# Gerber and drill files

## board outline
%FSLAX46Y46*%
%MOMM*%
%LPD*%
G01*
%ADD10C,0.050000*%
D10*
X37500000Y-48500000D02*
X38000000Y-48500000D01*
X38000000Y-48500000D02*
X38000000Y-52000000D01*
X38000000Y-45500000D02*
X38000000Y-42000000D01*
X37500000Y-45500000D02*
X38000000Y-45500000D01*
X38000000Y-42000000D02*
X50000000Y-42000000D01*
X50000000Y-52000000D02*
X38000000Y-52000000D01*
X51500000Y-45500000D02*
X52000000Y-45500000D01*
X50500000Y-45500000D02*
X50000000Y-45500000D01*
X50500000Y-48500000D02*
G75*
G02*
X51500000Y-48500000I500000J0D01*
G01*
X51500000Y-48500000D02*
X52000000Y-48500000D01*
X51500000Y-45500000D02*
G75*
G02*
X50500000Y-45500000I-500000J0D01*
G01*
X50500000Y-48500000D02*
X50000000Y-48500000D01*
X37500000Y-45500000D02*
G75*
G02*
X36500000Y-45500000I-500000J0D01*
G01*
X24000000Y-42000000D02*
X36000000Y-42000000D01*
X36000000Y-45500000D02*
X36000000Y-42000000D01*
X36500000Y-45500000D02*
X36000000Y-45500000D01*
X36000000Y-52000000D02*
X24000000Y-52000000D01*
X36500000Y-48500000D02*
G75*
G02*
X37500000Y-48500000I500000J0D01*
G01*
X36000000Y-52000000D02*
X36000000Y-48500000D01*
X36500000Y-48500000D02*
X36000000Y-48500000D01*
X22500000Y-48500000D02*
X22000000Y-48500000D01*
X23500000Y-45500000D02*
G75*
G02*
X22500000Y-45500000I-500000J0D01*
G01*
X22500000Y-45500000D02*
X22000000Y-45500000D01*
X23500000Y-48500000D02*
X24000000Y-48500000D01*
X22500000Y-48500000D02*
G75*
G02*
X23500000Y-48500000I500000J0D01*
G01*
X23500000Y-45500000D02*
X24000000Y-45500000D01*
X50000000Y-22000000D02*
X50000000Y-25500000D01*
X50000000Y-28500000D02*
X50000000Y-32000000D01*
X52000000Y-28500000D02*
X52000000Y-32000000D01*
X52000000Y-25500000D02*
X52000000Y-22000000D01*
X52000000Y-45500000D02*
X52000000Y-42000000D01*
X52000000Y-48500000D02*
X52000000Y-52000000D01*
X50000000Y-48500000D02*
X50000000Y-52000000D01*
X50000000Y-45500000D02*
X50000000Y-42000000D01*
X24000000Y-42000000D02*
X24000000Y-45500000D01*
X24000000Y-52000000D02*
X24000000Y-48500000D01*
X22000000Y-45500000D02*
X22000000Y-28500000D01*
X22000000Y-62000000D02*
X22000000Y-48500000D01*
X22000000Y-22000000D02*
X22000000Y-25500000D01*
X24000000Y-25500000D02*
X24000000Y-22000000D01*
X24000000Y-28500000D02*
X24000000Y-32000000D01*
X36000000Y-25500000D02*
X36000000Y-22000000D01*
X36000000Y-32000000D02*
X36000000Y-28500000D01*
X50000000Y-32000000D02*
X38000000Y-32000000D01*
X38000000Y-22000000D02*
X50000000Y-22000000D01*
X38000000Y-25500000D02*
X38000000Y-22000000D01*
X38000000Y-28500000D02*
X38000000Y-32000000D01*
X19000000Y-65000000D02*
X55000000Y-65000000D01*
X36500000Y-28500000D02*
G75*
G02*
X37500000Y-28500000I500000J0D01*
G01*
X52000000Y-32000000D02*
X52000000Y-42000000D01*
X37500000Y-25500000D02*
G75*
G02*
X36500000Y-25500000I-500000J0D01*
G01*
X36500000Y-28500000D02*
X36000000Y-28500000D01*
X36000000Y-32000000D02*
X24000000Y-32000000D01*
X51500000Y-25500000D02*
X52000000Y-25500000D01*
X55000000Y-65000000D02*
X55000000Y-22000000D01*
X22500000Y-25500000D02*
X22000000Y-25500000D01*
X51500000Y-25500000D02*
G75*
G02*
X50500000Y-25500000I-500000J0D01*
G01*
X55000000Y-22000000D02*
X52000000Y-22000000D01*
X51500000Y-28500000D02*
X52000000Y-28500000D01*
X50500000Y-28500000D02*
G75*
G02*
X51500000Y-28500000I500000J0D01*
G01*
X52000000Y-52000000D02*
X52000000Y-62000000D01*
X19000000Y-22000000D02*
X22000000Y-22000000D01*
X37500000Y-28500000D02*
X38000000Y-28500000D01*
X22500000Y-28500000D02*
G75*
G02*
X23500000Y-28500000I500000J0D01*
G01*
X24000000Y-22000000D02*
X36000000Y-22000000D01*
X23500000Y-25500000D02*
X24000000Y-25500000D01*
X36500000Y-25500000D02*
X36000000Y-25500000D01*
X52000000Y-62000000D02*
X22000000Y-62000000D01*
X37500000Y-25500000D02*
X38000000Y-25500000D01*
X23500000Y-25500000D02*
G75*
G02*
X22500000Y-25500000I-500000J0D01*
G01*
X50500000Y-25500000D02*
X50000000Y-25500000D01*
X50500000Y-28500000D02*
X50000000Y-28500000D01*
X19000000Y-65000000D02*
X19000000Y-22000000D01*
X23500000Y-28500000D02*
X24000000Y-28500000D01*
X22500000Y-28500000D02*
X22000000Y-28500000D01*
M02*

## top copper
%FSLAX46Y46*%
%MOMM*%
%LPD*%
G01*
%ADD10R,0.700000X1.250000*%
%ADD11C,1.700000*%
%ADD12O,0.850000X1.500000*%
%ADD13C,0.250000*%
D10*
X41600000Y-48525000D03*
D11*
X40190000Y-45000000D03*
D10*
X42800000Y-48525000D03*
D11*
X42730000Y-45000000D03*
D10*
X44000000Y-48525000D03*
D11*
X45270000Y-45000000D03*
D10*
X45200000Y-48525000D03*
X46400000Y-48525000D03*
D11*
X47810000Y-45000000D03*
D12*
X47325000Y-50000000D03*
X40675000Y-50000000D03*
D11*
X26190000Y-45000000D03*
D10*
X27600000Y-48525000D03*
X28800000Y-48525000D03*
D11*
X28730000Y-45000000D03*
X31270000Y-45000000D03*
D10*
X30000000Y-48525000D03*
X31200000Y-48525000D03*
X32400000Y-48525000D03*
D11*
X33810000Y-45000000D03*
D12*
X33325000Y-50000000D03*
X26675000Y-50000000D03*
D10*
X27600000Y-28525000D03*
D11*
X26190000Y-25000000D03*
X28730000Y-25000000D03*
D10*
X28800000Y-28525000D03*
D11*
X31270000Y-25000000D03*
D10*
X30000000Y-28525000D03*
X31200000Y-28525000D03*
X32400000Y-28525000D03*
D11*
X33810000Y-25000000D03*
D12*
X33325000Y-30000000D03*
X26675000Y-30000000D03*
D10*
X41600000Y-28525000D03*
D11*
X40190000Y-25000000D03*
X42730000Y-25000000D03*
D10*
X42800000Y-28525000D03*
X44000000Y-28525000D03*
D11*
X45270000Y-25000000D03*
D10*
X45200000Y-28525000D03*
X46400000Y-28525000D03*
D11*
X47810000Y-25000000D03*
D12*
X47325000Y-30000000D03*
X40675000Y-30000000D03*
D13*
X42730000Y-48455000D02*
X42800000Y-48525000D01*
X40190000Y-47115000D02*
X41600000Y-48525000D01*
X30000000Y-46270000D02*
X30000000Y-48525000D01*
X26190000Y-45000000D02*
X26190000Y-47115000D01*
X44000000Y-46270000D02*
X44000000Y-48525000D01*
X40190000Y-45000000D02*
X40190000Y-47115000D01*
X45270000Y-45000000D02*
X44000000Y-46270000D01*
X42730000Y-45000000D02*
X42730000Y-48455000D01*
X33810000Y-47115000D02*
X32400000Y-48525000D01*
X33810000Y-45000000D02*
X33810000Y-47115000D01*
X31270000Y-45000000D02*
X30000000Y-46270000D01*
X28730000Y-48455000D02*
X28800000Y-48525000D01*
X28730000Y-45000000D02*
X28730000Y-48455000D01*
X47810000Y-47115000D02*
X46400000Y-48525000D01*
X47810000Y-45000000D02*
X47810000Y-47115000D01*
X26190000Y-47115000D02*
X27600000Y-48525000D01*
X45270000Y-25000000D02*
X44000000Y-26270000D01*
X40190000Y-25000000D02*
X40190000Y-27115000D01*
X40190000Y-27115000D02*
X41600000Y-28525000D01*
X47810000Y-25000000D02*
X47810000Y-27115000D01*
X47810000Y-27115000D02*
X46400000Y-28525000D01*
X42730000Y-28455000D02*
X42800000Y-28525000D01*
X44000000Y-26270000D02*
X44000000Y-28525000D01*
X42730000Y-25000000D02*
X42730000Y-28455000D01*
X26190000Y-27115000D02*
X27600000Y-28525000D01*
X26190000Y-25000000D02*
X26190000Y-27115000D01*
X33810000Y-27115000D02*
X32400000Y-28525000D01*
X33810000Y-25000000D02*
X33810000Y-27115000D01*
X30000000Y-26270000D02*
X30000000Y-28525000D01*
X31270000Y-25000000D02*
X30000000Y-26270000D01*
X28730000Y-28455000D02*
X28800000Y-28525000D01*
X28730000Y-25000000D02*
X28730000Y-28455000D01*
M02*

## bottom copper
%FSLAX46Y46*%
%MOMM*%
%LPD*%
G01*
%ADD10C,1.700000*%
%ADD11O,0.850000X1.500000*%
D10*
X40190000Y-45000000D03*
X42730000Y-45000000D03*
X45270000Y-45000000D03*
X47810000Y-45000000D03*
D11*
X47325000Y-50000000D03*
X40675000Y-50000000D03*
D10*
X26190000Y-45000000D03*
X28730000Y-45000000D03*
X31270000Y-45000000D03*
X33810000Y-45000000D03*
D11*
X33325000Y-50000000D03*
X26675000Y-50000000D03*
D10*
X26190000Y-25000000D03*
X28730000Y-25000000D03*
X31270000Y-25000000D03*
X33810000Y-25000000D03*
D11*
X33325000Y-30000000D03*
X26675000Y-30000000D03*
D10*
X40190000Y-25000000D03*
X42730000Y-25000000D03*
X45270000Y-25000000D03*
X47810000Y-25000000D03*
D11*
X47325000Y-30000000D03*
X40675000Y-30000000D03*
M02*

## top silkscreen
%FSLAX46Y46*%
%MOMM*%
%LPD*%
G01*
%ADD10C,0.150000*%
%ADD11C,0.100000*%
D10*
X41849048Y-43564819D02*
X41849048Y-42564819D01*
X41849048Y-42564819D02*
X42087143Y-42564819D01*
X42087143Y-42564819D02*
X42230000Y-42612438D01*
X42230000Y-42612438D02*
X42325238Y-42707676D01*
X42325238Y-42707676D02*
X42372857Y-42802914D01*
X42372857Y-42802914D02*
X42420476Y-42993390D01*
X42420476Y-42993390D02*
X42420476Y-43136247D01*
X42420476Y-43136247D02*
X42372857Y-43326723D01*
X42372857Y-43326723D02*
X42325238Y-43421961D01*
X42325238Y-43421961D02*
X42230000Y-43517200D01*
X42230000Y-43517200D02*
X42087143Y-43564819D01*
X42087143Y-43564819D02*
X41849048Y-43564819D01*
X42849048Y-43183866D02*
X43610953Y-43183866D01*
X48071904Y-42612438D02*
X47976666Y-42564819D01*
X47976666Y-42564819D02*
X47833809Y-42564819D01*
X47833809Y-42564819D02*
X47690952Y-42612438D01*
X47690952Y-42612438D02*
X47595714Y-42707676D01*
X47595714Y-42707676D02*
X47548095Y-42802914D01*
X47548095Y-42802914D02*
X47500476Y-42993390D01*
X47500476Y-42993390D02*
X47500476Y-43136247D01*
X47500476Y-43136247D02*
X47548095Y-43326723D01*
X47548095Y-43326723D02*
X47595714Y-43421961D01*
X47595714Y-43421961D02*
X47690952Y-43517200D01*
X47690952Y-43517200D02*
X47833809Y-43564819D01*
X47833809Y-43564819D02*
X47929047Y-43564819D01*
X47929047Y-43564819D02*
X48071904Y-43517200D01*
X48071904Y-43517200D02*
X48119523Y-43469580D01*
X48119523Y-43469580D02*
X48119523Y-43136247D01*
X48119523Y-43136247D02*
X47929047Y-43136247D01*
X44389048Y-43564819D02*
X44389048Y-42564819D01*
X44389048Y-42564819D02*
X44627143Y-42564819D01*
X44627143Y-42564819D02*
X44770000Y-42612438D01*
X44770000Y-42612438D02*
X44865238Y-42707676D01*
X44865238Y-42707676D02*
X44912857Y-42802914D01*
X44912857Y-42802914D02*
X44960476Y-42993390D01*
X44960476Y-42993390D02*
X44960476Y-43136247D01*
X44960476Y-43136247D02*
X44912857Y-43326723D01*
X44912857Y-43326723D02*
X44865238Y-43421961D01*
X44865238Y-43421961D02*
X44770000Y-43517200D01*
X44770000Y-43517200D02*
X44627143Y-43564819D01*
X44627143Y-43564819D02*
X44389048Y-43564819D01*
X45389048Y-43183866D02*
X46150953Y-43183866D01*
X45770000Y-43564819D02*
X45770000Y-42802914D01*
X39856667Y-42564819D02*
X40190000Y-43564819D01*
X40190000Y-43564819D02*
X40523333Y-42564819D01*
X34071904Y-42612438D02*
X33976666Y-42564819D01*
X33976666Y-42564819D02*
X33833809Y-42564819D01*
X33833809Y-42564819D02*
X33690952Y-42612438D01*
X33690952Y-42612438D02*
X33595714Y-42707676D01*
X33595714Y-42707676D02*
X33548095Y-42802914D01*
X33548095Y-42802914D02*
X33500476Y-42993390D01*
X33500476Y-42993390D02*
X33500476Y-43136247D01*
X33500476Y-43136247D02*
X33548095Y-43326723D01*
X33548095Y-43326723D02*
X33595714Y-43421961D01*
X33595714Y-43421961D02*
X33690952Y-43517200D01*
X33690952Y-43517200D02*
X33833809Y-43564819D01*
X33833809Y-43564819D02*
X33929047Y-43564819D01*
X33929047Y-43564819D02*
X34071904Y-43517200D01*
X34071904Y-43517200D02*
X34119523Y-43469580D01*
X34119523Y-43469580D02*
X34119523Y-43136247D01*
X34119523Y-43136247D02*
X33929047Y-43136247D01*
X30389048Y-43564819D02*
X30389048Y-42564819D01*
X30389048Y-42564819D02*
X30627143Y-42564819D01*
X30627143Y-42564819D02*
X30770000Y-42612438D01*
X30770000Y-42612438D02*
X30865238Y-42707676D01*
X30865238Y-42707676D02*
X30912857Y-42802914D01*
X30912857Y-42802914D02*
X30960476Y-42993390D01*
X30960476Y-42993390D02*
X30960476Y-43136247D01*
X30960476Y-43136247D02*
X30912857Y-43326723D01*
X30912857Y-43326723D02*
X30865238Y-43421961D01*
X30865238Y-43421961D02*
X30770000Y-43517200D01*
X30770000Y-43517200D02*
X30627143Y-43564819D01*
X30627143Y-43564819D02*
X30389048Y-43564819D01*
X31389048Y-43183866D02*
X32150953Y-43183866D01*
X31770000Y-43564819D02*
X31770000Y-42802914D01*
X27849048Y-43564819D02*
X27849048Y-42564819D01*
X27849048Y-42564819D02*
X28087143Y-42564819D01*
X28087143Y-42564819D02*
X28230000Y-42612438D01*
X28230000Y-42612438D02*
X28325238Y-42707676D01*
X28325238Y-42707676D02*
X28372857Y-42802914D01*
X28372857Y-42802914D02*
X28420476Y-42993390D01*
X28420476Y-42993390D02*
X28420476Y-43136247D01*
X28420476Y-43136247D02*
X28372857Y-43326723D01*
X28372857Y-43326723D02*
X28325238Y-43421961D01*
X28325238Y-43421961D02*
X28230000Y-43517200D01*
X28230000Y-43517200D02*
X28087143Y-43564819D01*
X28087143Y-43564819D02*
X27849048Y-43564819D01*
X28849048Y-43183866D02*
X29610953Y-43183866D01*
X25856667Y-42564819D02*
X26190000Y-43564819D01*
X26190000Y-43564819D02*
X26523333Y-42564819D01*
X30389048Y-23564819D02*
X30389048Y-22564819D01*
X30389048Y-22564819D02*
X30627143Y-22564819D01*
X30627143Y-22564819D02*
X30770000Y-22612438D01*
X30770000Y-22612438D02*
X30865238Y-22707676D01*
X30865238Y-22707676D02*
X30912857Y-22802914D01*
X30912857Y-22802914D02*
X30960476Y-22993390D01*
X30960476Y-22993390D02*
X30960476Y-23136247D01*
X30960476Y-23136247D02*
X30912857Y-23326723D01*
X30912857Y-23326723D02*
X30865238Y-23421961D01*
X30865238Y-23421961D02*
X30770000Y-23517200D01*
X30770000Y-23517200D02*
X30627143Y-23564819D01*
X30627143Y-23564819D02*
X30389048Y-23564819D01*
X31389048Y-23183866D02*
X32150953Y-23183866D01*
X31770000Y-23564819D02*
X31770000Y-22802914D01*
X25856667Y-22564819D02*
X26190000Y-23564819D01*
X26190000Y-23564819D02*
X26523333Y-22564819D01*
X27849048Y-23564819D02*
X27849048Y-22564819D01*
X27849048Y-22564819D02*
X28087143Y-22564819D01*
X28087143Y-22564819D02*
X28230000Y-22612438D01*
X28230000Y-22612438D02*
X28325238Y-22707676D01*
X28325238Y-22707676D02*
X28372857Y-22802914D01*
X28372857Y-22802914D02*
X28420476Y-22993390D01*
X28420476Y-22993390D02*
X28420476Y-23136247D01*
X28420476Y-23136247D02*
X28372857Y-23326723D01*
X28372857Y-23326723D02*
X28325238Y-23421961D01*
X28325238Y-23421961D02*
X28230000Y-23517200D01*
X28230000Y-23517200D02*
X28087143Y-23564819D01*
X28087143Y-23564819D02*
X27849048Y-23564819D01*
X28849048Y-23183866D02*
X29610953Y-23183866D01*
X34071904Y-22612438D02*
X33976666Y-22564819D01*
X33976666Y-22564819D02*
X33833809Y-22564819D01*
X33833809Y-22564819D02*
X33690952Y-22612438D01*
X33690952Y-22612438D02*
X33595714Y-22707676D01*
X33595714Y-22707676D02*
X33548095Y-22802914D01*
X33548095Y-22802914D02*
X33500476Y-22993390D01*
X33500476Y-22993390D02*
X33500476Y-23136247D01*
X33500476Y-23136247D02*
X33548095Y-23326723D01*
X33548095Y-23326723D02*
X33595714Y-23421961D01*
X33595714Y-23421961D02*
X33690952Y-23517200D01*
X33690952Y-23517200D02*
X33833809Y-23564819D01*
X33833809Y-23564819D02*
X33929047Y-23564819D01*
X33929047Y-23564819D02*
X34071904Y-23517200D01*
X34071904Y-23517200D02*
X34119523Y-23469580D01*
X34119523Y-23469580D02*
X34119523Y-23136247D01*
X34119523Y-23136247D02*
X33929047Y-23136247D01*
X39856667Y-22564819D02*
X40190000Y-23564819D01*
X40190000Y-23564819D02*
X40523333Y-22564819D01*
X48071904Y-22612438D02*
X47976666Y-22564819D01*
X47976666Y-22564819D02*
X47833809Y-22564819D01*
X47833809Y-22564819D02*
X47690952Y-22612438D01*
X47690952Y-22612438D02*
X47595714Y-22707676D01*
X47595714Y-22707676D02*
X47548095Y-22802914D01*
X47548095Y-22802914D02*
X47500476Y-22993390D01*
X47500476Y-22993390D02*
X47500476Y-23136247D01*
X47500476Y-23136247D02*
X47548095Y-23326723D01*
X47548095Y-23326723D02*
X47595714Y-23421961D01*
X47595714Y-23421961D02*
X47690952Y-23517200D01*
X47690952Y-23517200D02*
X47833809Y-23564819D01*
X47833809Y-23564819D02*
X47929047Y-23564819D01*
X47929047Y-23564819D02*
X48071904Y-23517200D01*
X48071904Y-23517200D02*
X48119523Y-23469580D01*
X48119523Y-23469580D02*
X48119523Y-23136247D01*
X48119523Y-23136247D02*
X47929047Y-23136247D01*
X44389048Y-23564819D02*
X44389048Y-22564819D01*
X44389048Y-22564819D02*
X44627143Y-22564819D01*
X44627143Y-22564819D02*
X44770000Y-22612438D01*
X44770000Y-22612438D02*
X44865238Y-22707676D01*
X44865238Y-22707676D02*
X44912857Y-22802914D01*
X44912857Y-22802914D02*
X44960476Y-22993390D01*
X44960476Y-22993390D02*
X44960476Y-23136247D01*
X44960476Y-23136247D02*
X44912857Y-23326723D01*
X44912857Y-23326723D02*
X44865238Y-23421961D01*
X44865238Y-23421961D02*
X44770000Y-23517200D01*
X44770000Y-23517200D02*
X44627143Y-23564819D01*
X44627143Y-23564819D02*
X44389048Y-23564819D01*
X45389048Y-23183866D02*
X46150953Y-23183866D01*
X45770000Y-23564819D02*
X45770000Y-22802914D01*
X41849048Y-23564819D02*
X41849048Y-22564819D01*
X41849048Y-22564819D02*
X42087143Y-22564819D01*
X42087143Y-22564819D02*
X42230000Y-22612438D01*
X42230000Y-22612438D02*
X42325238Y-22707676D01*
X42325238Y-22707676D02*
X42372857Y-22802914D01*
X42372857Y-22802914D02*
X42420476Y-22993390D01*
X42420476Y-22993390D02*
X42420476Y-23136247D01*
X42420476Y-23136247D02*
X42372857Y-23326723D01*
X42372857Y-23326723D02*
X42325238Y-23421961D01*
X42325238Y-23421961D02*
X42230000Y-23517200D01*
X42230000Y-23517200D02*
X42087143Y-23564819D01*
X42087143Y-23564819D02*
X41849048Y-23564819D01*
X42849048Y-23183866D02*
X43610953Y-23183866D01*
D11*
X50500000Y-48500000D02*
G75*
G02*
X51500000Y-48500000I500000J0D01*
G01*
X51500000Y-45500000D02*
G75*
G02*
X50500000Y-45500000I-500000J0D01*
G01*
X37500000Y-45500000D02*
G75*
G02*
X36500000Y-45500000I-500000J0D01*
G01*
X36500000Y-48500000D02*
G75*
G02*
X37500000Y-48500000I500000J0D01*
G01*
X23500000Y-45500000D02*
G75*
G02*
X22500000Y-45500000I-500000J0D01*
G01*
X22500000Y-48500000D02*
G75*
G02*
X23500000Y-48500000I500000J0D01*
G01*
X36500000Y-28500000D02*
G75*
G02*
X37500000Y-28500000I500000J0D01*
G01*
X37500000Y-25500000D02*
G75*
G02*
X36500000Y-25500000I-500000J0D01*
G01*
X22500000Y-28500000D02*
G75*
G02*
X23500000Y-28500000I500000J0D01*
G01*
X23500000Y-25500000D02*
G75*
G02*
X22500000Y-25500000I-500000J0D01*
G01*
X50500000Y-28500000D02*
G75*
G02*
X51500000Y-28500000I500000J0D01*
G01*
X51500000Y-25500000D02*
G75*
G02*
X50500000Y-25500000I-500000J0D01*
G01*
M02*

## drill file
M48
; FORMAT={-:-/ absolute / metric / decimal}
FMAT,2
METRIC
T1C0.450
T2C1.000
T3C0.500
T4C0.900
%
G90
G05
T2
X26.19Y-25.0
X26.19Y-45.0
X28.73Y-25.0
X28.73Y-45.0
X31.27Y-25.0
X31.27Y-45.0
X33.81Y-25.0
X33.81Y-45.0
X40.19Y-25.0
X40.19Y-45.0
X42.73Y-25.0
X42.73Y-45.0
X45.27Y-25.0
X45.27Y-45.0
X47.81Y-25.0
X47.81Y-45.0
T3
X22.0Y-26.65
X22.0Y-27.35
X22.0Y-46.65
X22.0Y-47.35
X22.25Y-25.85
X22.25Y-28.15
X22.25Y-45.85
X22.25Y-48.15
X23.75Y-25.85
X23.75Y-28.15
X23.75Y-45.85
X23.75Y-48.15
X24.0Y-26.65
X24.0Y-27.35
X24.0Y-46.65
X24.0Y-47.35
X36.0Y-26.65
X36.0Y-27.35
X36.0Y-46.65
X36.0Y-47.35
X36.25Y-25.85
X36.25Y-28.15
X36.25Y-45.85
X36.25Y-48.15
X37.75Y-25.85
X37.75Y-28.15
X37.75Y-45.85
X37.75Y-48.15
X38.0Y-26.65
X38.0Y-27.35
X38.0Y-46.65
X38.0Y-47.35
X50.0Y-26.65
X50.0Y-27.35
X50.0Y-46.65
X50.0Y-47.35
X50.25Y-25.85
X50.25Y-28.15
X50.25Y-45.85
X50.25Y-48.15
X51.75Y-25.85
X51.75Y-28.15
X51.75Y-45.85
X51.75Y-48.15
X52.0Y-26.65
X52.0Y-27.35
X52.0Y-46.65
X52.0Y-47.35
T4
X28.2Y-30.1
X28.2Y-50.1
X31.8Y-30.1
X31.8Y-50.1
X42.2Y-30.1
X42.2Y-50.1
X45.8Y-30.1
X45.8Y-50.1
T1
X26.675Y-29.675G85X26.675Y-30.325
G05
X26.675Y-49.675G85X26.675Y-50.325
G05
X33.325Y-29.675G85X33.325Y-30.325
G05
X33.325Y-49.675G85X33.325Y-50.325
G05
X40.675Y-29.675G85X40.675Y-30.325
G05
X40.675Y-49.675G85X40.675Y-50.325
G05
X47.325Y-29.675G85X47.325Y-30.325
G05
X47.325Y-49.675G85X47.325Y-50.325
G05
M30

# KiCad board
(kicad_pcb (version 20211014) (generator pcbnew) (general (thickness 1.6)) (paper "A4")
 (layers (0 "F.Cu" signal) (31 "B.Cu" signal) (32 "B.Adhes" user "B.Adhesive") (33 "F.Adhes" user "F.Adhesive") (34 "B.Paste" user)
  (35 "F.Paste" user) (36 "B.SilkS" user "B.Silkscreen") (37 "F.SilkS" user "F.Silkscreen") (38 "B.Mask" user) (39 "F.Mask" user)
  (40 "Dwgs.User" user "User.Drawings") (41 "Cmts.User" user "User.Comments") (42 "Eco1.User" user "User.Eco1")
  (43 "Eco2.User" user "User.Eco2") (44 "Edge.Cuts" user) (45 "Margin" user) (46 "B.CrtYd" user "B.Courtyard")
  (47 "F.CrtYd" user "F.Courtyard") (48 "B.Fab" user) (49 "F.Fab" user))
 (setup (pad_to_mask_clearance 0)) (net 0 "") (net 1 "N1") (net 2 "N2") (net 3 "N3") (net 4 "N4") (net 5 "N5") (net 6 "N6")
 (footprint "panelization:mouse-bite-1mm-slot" (layer "F.Cu") (at 51 47 90)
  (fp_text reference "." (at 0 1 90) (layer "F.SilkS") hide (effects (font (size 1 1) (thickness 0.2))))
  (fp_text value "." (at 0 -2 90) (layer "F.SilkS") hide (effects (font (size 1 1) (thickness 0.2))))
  (fp_arc (start -1.5 -0.5) (mid -1 0) (end -1.5 0.5) (layer "F.SilkS") (width 0.1))
  (fp_arc (start 1.5 0.5) (mid 1 0) (end 1.5 -0.5) (layer "F.SilkS") (width 0.1))
  (pad "" np_thru_hole circle locked (at -1.15 -0.75 90) (size 0.5 0.5) (drill 0.5) (layers *.Cu *.Mask))
  (pad "" np_thru_hole circle locked (at -0.35 1 90) (size 0.5 0.5) (drill 0.5) (layers *.Cu *.Mask))
  (pad "" np_thru_hole circle locked (at -0.35 -1 90) (size 0.5 0.5) (drill 0.5) (layers *.Cu *.Mask))
  (pad "" np_thru_hole circle locked (at 0.35 -1 90) (size 0.5 0.5) (drill 0.5) (layers *.Cu *.Mask))
  (pad "" np_thru_hole circle locked (at 1.15 -0.75 90) (size 0.5 0.5) (drill 0.5) (layers *.Cu *.Mask))
  (pad "" np_thru_hole circle locked (at 1.15 0.75 90) (size 0.5 0.5) (drill 0.5) (layers *.Cu *.Mask))
  (pad "" np_thru_hole circle locked (at -1.15 0.75 90) (size 0.5 0.5) (drill 0.5) (layers *.Cu *.Mask))
  (pad "" np_thru_hole circle locked (at 0.35 1 90) (size 0.5 0.5) (drill 0.5) (layers *.Cu *.Mask)))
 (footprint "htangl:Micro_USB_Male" (layer "F.Cu") (at 44 50)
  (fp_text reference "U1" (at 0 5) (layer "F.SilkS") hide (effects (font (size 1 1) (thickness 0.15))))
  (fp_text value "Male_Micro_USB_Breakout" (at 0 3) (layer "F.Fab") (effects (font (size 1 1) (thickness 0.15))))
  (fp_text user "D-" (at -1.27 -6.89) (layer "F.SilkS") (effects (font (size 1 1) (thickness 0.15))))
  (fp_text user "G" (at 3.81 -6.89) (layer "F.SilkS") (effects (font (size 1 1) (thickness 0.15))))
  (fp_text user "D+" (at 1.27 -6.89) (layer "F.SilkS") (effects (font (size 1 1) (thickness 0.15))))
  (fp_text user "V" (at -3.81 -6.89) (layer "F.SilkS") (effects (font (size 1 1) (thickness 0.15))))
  (pad "" np_thru_hole circle (at -1.8 0.1) (size 0.9 0.9) (drill 0.9) (layers *.Cu *.Mask))
  (pad "" np_thru_hole circle (at 1.8 0.1) (size 0.9 0.9) (drill 0.9) (layers *.Cu *.Mask))
  (pad "1" smd rect (at -2.4 -1.475) (size 0.7 1.25) (layers "F.Cu" "F.Paste" "F.Mask"))
  (pad "1" thru_hole circle (at -3.81 -5) (size 1.7 1.7) (drill 1) (layers *.Cu *.Mask))
  (pad "2" smd rect (at -1.2 -1.475) (size 0.7 1.25) (layers "F.Cu" "F.Paste" "F.Mask"))
  (pad "2" thru_hole circle (at -1.27 -5) (size 1.7 1.7) (drill 1) (layers *.Cu *.Mask))
  (pad "3" smd rect (at 0 -1.475) (size 0.7 1.25) (layers "F.Cu" "F.Paste" "F.Mask"))
  (pad "3" thru_hole circle (at 1.27 -5) (size 1.7 1.7) (drill 1) (layers *.Cu *.Mask))
  (pad "4" smd rect (at 1.2 -1.475) (size 0.7 1.25) (layers "F.Cu" "F.Paste" "F.Mask"))
  (pad "5" smd rect (at 2.4 -1.475) (size 0.7 1.25) (layers "F.Cu" "F.Paste" "F.Mask"))
  (pad "5" thru_hole circle (at 3.81 -5) (size 1.7 1.7) (drill 1) (layers *.Cu *.Mask))
  (pad "6" thru_hole oval (at 3.325 0) (size 0.85 1.5) (drill oval 0.45 1.1) (layers *.Cu *.Mask))
  (pad "6" thru_hole oval (at -3.325 0) (size 0.85 1.5) (drill oval 0.45 1.1) (layers *.Cu *.Mask)))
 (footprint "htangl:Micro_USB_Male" (layer "F.Cu") (at 30 50)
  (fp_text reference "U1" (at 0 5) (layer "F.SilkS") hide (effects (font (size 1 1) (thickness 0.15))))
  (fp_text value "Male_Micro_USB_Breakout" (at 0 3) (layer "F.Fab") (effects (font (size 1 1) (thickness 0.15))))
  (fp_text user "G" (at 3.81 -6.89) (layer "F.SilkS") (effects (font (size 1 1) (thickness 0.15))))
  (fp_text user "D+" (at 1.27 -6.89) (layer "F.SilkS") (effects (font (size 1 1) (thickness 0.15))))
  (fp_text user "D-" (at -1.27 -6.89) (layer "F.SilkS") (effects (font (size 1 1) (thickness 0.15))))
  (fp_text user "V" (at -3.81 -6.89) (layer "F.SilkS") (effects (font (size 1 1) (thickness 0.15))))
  (pad "" np_thru_hole circle (at 1.8 0.1) (size 0.9 0.9) (drill 0.9) (layers *.Cu *.Mask))
  (pad "" np_thru_hole circle (at -1.8 0.1) (size 0.9 0.9) (drill 0.9) (layers *.Cu *.Mask))
  (pad "1" thru_hole circle (at -3.81 -5) (size 1.7 1.7) (drill 1) (layers *.Cu *.Mask))
  (pad "1" smd rect (at -2.4 -1.475) (size 0.7 1.25) (layers "F.Cu" "F.Paste" "F.Mask"))
  (pad "2" smd rect (at -1.2 -1.475) (size 0.7 1.25) (layers "F.Cu" "F.Paste" "F.Mask"))
  (pad "2" thru_hole circle (at -1.27 -5) (size 1.7 1.7) (drill 1) (layers *.Cu *.Mask))
  (pad "3" thru_hole circle (at 1.27 -5) (size 1.7 1.7) (drill 1) (layers *.Cu *.Mask))
  (pad "3" smd rect (at 0 -1.475) (size 0.7 1.25) (layers "F.Cu" "F.Paste" "F.Mask"))
  (pad "4" smd rect (at 1.2 -1.475) (size 0.7 1.25) (layers "F.Cu" "F.Paste" "F.Mask"))
  (pad "5" smd rect (at 2.4 -1.475) (size 0.7 1.25) (layers "F.Cu" "F.Paste" "F.Mask"))
  (pad "5" thru_hole circle (at 3.81 -5) (size 1.7 1.7) (drill 1) (layers *.Cu *.Mask))
  (pad "6" thru_hole oval (at 3.325 0) (size 0.85 1.5) (drill oval 0.45 1.1) (layers *.Cu *.Mask))
  (pad "6" thru_hole oval (at -3.325 0) (size 0.85 1.5) (drill oval 0.45 1.1) (layers *.Cu *.Mask)))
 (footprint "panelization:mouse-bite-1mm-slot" (layer "F.Cu") (at 37 47 90)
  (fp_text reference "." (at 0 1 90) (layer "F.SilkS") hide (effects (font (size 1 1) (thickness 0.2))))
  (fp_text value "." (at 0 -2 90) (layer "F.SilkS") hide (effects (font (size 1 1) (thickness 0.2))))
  (fp_arc (start 1.5 0.5) (mid 1 0) (end 1.5 -0.5) (layer "F.SilkS") (width 0.1))
  (fp_arc (start -1.5 -0.5) (mid -1 0) (end -1.5 0.5) (layer "F.SilkS") (width 0.1))
  (pad "" np_thru_hole circle locked (at -0.35 -1 90) (size 0.5 0.5) (drill 0.5) (layers *.Cu *.Mask))
  (pad "" np_thru_hole circle locked (at -0.35 1 90) (size 0.5 0.5) (drill 0.5) (layers *.Cu *.Mask))
  (pad "" np_thru_hole circle locked (at 1.15 -0.75 90) (size 0.5 0.5) (drill 0.5) (layers *.Cu *.Mask))
  (pad "" np_thru_hole circle locked (at -1.15 -0.75 90) (size 0.5 0.5) (drill 0.5) (layers *.Cu *.Mask))
  (pad "" np_thru_hole circle locked (at 1.15 0.75 90) (size 0.5 0.5) (drill 0.5) (layers *.Cu *.Mask))
  (pad "" np_thru_hole circle locked (at -1.15 0.75 90) (size 0.5 0.5) (drill 0.5) (layers *.Cu *.Mask))
  (pad "" np_thru_hole circle locked (at 0.35 -1 90) (size 0.5 0.5) (drill 0.5) (layers *.Cu *.Mask))
  (pad "" np_thru_hole circle locked (at 0.35 1 90) (size 0.5 0.5) (drill 0.5) (layers *.Cu *.Mask)))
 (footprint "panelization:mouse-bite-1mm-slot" (layer "F.Cu") (at 23 47 90)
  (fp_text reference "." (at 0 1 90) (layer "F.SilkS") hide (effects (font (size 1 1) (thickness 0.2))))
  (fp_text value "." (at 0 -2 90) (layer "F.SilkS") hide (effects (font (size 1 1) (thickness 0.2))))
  (fp_arc (start 1.5 0.5) (mid 1 0) (end 1.5 -0.5) (layer "F.SilkS") (width 0.1))
  (fp_arc (start -1.5 -0.5) (mid -1 0) (end -1.5 0.5) (layer "F.SilkS") (width 0.1))
  (pad "" np_thru_hole circle locked (at 0.35 1 90) (size 0.5 0.5) (drill 0.5) (layers *.Cu *.Mask))
  (pad "" np_thru_hole circle locked (at -0.35 -1 90) (size 0.5 0.5) (drill 0.5) (layers *.Cu *.Mask))
  (pad "" np_thru_hole circle locked (at 1.15 -0.75 90) (size 0.5 0.5) (drill 0.5) (layers *.Cu *.Mask))
  (pad "" np_thru_hole circle locked (at 1.15 0.75 90) (size 0.5 0.5) (drill 0.5) (layers *.Cu *.Mask))
  (pad "" np_thru_hole circle locked (at -1.15 0.75 90) (size 0.5 0.5) (drill 0.5) (layers *.Cu *.Mask))
  (pad "" np_thru_hole circle locked (at -1.15 -0.75 90) (size 0.5 0.5) (drill 0.5) (layers *.Cu *.Mask))
  (pad "" np_thru_hole circle locked (at 0.35 -1 90) (size 0.5 0.5) (drill 0.5) (layers *.Cu *.Mask))
  (pad "" np_thru_hole circle locked (at -0.35 1 90) (size 0.5 0.5) (drill 0.5) (layers *.Cu *.Mask)))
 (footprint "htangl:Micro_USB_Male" (layer "F.Cu") (at 30 30)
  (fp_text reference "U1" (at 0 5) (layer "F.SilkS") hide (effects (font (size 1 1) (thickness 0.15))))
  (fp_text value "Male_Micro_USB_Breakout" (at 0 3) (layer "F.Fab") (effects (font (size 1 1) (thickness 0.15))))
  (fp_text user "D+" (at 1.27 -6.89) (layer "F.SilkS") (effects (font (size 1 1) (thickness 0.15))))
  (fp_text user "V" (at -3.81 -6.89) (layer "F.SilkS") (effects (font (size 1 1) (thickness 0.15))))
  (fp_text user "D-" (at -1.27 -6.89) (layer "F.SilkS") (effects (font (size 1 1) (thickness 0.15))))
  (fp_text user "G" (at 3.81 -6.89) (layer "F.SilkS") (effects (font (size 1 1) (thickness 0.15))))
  (pad "" np_thru_hole circle (at 1.8 0.1) (size 0.9 0.9) (drill 0.9) (layers *.Cu *.Mask))
  (pad "" np_thru_hole circle (at -1.8 0.1) (size 0.9 0.9) (drill 0.9) (layers *.Cu *.Mask))
  (pad "1" smd rect (at -2.4 -1.475) (size 0.7 1.25) (layers "F.Cu" "F.Paste" "F.Mask") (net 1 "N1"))
  (pad "1" thru_hole circle (at -3.81 -5) (size 1.7 1.7) (drill 1) (layers *.Cu *.Mask) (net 1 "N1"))
  (pad "2" thru_hole circle (at -1.27 -5) (size 1.7 1.7) (drill 1) (layers *.Cu *.Mask) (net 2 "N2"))
  (pad "2" smd rect (at -1.2 -1.475) (size 0.7 1.25) (layers "F.Cu" "F.Paste" "F.Mask") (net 2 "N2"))
  (pad "3" thru_hole circle (at 1.27 -5) (size 1.7 1.7) (drill 1) (layers *.Cu *.Mask) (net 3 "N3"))
  (pad "3" smd rect (at 0 -1.475) (size 0.7 1.25) (layers "F.Cu" "F.Paste" "F.Mask") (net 3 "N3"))
  (pad "4" smd rect (at 1.2 -1.475) (size 0.7 1.25) (layers "F.Cu" "F.Paste" "F.Mask") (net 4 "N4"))
  (pad "5" smd rect (at 2.4 -1.475) (size 0.7 1.25) (layers "F.Cu" "F.Paste" "F.Mask") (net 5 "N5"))
  (pad "5" thru_hole circle (at 3.81 -5) (size 1.7 1.7) (drill 1) (layers *.Cu *.Mask) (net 5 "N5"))
  (pad "6" thru_hole oval (at 3.325 0) (size 0.85 1.5) (drill oval 0.45 1.1) (layers *.Cu *.Mask) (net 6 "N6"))
  (pad "6" thru_hole oval (at -3.325 0) (size 0.85 1.5) (drill oval 0.45 1.1) (layers *.Cu *.Mask) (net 6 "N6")))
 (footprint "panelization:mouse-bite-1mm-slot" (layer "F.Cu") (at 37 27 90)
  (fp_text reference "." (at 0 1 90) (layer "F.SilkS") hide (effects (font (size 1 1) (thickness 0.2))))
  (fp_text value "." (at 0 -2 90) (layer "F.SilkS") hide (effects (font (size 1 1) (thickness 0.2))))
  (fp_arc (start -1.5 -0.5) (mid -1 0) (end -1.5 0.5) (layer "F.SilkS") (width 0.1))
  (fp_arc (start 1.5 0.5) (mid 1 0) (end 1.5 -0.5) (layer "F.SilkS") (width 0.1))
  (pad "" np_thru_hole circle locked (at 1.15 -0.75 90) (size 0.5 0.5) (drill 0.5) (layers *.Cu *.Mask))
  (pad "" np_thru_hole circle locked (at -0.35 -1 90) (size 0.5 0.5) (drill 0.5) (layers *.Cu *.Mask))
  (pad "" np_thru_hole circle locked (at -0.35 1 90) (size 0.5 0.5) (drill 0.5) (layers *.Cu *.Mask))
  (pad "" np_thru_hole circle locked (at -1.15 -0.75 90) (size 0.5 0.5) (drill 0.5) (layers *.Cu *.Mask))
  (pad "" np_thru_hole circle locked (at 1.15 0.75 90) (size 0.5 0.5) (drill 0.5) (layers *.Cu *.Mask))
  (pad "" np_thru_hole circle locked (at 0.35 1 90) (size 0.5 0.5) (drill 0.5) (layers *.Cu *.Mask))
  (pad "" np_thru_hole circle locked (at -1.15 0.75 90) (size 0.5 0.5) (drill 0.5) (layers *.Cu *.Mask))
  (pad "" np_thru_hole circle locked (at 0.35 -1 90) (size 0.5 0.5) (drill 0.5) (layers *.Cu *.Mask)))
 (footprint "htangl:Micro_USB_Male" (layer "F.Cu") (at 44 30)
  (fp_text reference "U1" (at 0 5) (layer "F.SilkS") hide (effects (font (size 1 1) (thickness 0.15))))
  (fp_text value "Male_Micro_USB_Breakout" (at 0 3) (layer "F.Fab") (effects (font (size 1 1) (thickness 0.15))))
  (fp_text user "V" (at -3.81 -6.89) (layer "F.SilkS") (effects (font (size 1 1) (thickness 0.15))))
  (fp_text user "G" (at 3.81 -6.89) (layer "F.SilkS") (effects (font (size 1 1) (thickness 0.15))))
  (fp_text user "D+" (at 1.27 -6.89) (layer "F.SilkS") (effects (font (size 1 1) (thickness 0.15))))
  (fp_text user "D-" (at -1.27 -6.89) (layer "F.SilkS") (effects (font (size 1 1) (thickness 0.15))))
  (pad "" np_thru_hole circle (at -1.8 0.1) (size 0.9 0.9) (drill 0.9) (layers *.Cu *.Mask))
  (pad "" np_thru_hole circle (at 1.8 0.1) (size 0.9 0.9) (drill 0.9) (layers *.Cu *.Mask))
  (pad "1" smd rect (at -2.4 -1.475) (size 0.7 1.25) (layers "F.Cu" "F.Paste" "F.Mask"))
  (pad "1" thru_hole circle (at -3.81 -5) (size 1.7 1.7) (drill 1) (layers *.Cu *.Mask))
  (pad "2" thru_hole circle (at -1.27 -5) (size 1.7 1.7) (drill 1) (layers *.Cu *.Mask))
  (pad "2" smd rect (at -1.2 -1.475) (size 0.7 1.25) (layers "F.Cu" "F.Paste" "F.Mask"))
  (pad "3" smd rect (at 0 -1.475) (size 0.7 1.25) (layers "F.Cu" "F.Paste" "F.Mask"))
  (pad "3" thru_hole circle (at 1.27 -5) (size 1.7 1.7) (drill 1) (layers *.Cu *.Mask))
  (pad "4" smd rect (at 1.2 -1.475) (size 0.7 1.25) (layers "F.Cu" "F.Paste" "F.Mask"))
  (pad "5" smd rect (at 2.4 -1.475) (size 0.7 1.25) (layers "F.Cu" "F.Paste" "F.Mask"))
  (pad "5" thru_hole circle (at 3.81 -5) (size 1.7 1.7) (drill 1) (layers *.Cu *.Mask))
  (pad "6" thru_hole oval (at 3.325 0) (size 0.85 1.5) (drill oval 0.45 1.1) (layers *.Cu *.Mask))
  (pad "6" thru_hole oval (at -3.325 0) (size 0.85 1.5) (drill oval 0.45 1.1) (layers *.Cu *.Mask)))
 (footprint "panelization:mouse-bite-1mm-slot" (layer "F.Cu") (at 23 27 90)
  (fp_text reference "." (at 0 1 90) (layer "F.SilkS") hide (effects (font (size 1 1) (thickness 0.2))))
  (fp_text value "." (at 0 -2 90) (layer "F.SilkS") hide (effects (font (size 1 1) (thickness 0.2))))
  (fp_arc (start -1.5 -0.5) (mid -1 0) (end -1.5 0.5) (layer "F.SilkS") (width 0.1))
  (fp_arc (start 1.5 0.5) (mid 1 0) (end 1.5 -0.5) (layer "F.SilkS") (width 0.1))
  (pad "" np_thru_hole circle locked (at 0.35 -1 90) (size 0.5 0.5) (drill 0.5) (layers *.Cu *.Mask))
  (pad "" np_thru_hole circle locked (at -0.35 -1 90) (size 0.5 0.5) (drill 0.5) (layers *.Cu *.Mask))
  (pad "" np_thru_hole circle locked (at 0.35 1 90) (size 0.5 0.5) (drill 0.5) (layers *.Cu *.Mask))
  (pad "" np_thru_hole circle locked (at -0.35 1 90) (size 0.5 0.5) (drill 0.5) (layers *.Cu *.Mask))
  (pad "" np_thru_hole circle locked (at -1.15 0.75 90) (size 0.5 0.5) (drill 0.5) (layers *.Cu *.Mask))
  (pad "" np_thru_hole circle locked (at 1.15 -0.75 90) (size 0.5 0.5) (drill 0.5) (layers *.Cu *.Mask))
  (pad "" np_thru_hole circle locked (at -1.15 -0.75 90) (size 0.5 0.5) (drill 0.5) (layers *.Cu *.Mask))
  (pad "" np_thru_hole circle locked (at 1.15 0.75 90) (size 0.5 0.5) (drill 0.5) (layers *.Cu *.Mask)))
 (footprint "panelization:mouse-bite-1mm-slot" (layer "F.Cu") (at 51 27 90)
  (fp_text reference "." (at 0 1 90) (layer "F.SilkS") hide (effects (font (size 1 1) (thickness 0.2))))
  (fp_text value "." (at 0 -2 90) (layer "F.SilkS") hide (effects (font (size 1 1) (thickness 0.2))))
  (fp_arc (start -1.5 -0.5) (mid -1 0) (end -1.5 0.5) (layer "F.SilkS") (width 0.1))
  (fp_arc (start 1.5 0.5) (mid 1 0) (end 1.5 -0.5) (layer "F.SilkS") (width 0.1))
  (pad "" np_thru_hole circle locked (at 0.35 -1 90) (size 0.5 0.5) (drill 0.5) (layers *.Cu *.Mask))
  (pad "" np_thru_hole circle locked (at -0.35 1 90) (size 0.5 0.5) (drill 0.5) (layers *.Cu *.Mask))
  (pad "" np_thru_hole circle locked (at 1.15 0.75 90) (size 0.5 0.5) (drill 0.5) (layers *.Cu *.Mask))
  (pad "" np_thru_hole circle locked (at 1.15 -0.75 90) (size 0.5 0.5) (drill 0.5) (layers *.Cu *.Mask))
  (pad "" np_thru_hole circle locked (at -1.15 -0.75 90) (size 0.5 0.5) (drill 0.5) (layers *.Cu *.Mask))
  (pad "" np_thru_hole circle locked (at -0.35 -1 90) (size 0.5 0.5) (drill 0.5) (layers *.Cu *.Mask))
  (pad "" np_thru_hole circle locked (at -1.15 0.75 90) (size 0.5 0.5) (drill 0.5) (layers *.Cu *.Mask))
  (pad "" np_thru_hole circle locked (at 0.35 1 90) (size 0.5 0.5) (drill 0.5) (layers *.Cu *.Mask)))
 (gr_line (start 37.5 48.5) (end 38 48.5) (layer "Edge.Cuts") (width 0.05))
 (gr_line (start 38 48.5) (end 38 52) (layer "Edge.Cuts") (width 0.05))
 (gr_line (start 38 45.5) (end 38 42) (layer "Edge.Cuts") (width 0.05))
 (gr_line (start 37.5 45.5) (end 38 45.5) (layer "Edge.Cuts") (width 0.05))
 (gr_line (start 38 42) (end 50 42) (layer "Edge.Cuts") (width 0.05))
 (gr_line (start 50 52) (end 38 52) (layer "Edge.Cuts") (width 0.05))
 (gr_line (start 51.5 45.5) (end 52 45.5) (layer "Edge.Cuts") (width 0.05))
 (gr_line (start 50.5 45.5) (end 50 45.5) (layer "Edge.Cuts") (width 0.05))
 (gr_arc (start 50.5 48.5) (mid 51 48) (end 51.5 48.5) (layer "Edge.Cuts") (width 0.05))
 (gr_line (start 51.5 48.5) (end 52 48.5) (layer "Edge.Cuts") (width 0.05))
 (gr_arc (start 51.5 45.5) (mid 51 46) (end 50.5 45.5) (layer "Edge.Cuts") (width 0.05))
 (gr_line (start 50.5 48.5) (end 50 48.5) (layer "Edge.Cuts") (width 0.05))
 (gr_arc (start 37.5 45.5) (mid 37 46) (end 36.5 45.5) (layer "Edge.Cuts") (width 0.05))
 (gr_line (start 24 42) (end 36 42) (layer "Edge.Cuts") (width 0.05))
 (gr_line (start 36 45.5) (end 36 42) (layer "Edge.Cuts") (width 0.05))
 (gr_line (start 36.5 45.5) (end 36 45.5) (layer "Edge.Cuts") (width 0.05))
 (gr_line (start 36 52) (end 24 52) (layer "Edge.Cuts") (width 0.05))
 (gr_arc (start 36.5 48.5) (mid 37 48) (end 37.5 48.5) (layer "Edge.Cuts") (width 0.05))
 (gr_line (start 36 52) (end 36 48.5) (layer "Edge.Cuts") (width 0.05))
 (gr_line (start 36.5 48.5) (end 36 48.5) (layer "Edge.Cuts") (width 0.05))
 (gr_line (start 22.5 48.5) (end 22 48.5) (layer "Edge.Cuts") (width 0.05))
 (gr_arc (start 23.5 45.5) (mid 23 46) (end 22.5 45.5) (layer "Edge.Cuts") (width 0.05))
 (gr_line (start 22.5 45.5) (end 22 45.5) (layer "Edge.Cuts") (width 0.05))
 (gr_line (start 23.5 48.5) (end 24 48.5) (layer "Edge.Cuts") (width 0.05))
 (gr_arc (start 22.5 48.5) (mid 23 48) (end 23.5 48.5) (layer "Edge.Cuts") (width 0.05))
 (gr_line (start 23.5 45.5) (end 24 45.5) (layer "Edge.Cuts") (width 0.05))
 (gr_line (start 50 22) (end 50 25.5) (layer "Edge.Cuts") (width 0.05))
 (gr_line (start 50 28.5) (end 50 32) (layer "Edge.Cuts") (width 0.05))
 (gr_line (start 52 28.5) (end 52 32) (layer "Edge.Cuts") (width 0.05))
 (gr_line (start 52 25.5) (end 52 22) (layer "Edge.Cuts") (width 0.05))
 (gr_line (start 52 45.5) (end 52 42) (layer "Edge.Cuts") (width 0.05))
 (gr_line (start 52 48.5) (end 52 52) (layer "Edge.Cuts") (width 0.05))
 (gr_line (start 50 48.5) (end 50 52) (layer "Edge.Cuts") (width 0.05))
 (gr_line (start 50 45.5) (end 50 42) (layer "Edge.Cuts") (width 0.05))
 (gr_line (start 24 42) (end 24 45.5) (layer "Edge.Cuts") (width 0.05))
 (gr_line (start 24 52) (end 24 48.5) (layer "Edge.Cuts") (width 0.05))
 (gr_line (start 22 45.5) (end 22 28.5) (layer "Edge.Cuts") (width 0.05))
 (gr_line (start 22 62) (end 22 48.5) (layer "Edge.Cuts") (width 0.05))
 (gr_line (start 22 22) (end 22 25.5) (layer "Edge.Cuts") (width 0.05))
 (gr_line (start 24 25.5) (end 24 22) (layer "Edge.Cuts") (width 0.05))
 (gr_line (start 24 28.5) (end 24 32) (layer "Edge.Cuts") (width 0.05))
 (gr_line (start 36 25.5) (end 36 22) (layer "Edge.Cuts") (width 0.05))
 (gr_line (start 36 32) (end 36 28.5) (layer "Edge.Cuts") (width 0.05))
 (gr_line (start 50 32) (end 38 32) (layer "Edge.Cuts") (width 0.05))
 (gr_line (start 38 22) (end 50 22) (layer "Edge.Cuts") (width 0.05))
 (gr_line (start 38 25.5) (end 38 22) (layer "Edge.Cuts") (width 0.05))
 (gr_line (start 38 28.5) (end 38 32) (layer "Edge.Cuts") (width 0.05))
 (gr_line (start 19 65) (end 55 65) (layer "Edge.Cuts") (width 0.05))
 (gr_arc (start 36.5 28.5) (mid 37 28) (end 37.5 28.5) (layer "Edge.Cuts") (width 0.05))
 (gr_line (start 52 32) (end 52 42) (layer "Edge.Cuts") (width 0.05))
 (gr_arc (start 37.5 25.5) (mid 37 26) (end 36.5 25.5) (layer "Edge.Cuts") (width 0.05))
 (gr_line (start 36.5 28.5) (end 36 28.5) (layer "Edge.Cuts") (width 0.05))
 (gr_line (start 36 32) (end 24 32) (layer "Edge.Cuts") (width 0.05))
 (gr_line (start 51.5 25.5) (end 52 25.5) (layer "Edge.Cuts") (width 0.05))
 (gr_line (start 55 65) (end 55 22) (layer "Edge.Cuts") (width 0.05))
 (gr_line (start 22.5 25.5) (end 22 25.5) (layer "Edge.Cuts") (width 0.05))
 (gr_arc (start 51.5 25.5) (mid 51 26) (end 50.5 25.5) (layer "Edge.Cuts") (width 0.05))
 (gr_line (start 55 22) (end 52 22) (layer "Edge.Cuts") (width 0.05))
 (gr_line (start 51.5 28.5) (end 52 28.5) (layer "Edge.Cuts") (width 0.05))
 (gr_arc (start 50.5 28.5) (mid 51 28) (end 51.5 28.5) (layer "Edge.Cuts") (width 0.05))
 (gr_line (start 52 52) (end 52 62) (layer "Edge.Cuts") (width 0.05))
 (gr_line (start 19 22) (end 22 22) (layer "Edge.Cuts") (width 0.05))
 (gr_line (start 37.5 28.5) (end 38 28.5) (layer "Edge.Cuts") (width 0.05))
 (gr_arc (start 22.5 28.5) (mid 23 28) (end 23.5 28.5) (layer "Edge.Cuts") (width 0.05))
 (gr_line (start 24 22) (end 36 22) (layer "Edge.Cuts") (width 0.05))
 (gr_line (start 23.5 25.5) (end 24 25.5) (layer "Edge.Cuts") (width 0.05))
 (gr_line (start 36.5 25.5) (end 36 25.5) (layer "Edge.Cuts") (width 0.05))
 (gr_line (start 52 62) (end 22 62) (layer "Edge.Cuts") (width 0.05))
 (gr_line (start 37.5 25.5) (end 38 25.5) (layer "Edge.Cuts") (width 0.05))
 (gr_arc (start 23.5 25.5) (mid 23 26) (end 22.5 25.5) (layer "Edge.Cuts") (width 0.05))
 (gr_line (start 50.5 25.5) (end 50 25.5) (layer "Edge.Cuts") (width 0.05))
 (gr_line (start 50.5 28.5) (end 50 28.5) (layer "Edge.Cuts") (width 0.05))
 (gr_line (start 19 65) (end 19 22) (layer "Edge.Cuts") (width 0.05))
 (gr_line (start 23.5 28.5) (end 24 28.5) (layer "Edge.Cuts") (width 0.05))
 (gr_line (start 22.5 28.5) (end 22 28.5) (layer "Edge.Cuts") (width 0.05))
 (segment (start 42.73 48.455) (end 42.8 48.525) (width 0.25) (layer "F.Cu") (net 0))
 (segment (start 40.19 47.115) (end 41.6 48.525) (width 0.25) (layer "F.Cu") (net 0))
 (segment (start 30 46.27) (end 30 48.525) (width 0.25) (layer "F.Cu") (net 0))
 (segment (start 26.19 45) (end 26.19 47.115) (width 0.25) (layer "F.Cu") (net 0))
 (segment (start 44 46.27) (end 44 48.525) (width 0.25) (layer "F.Cu") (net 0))
 (segment (start 40.19 45) (end 40.19 47.115) (width 0.25) (layer "F.Cu") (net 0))
 (segment (start 45.27 45) (end 44 46.27) (width 0.25) (layer "F.Cu") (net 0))
 (segment (start 42.73 45) (end 42.73 48.455) (width 0.25) (layer "F.Cu") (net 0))
 (segment (start 33.81 47.115) (end 32.4 48.525) (width 0.25) (layer "F.Cu") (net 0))
 (segment (start 33.81 45) (end 33.81 47.115) (width 0.25) (layer "F.Cu") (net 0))
 (segment (start 31.27 45) (end 30 46.27) (width 0.25) (layer "F.Cu") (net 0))
 (segment (start 28.73 48.455) (end 28.8 48.525) (width 0.25) (layer "F.Cu") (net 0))
 (segment (start 28.73 45) (end 28.73 48.455) (width 0.25) (layer "F.Cu") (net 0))
 (segment (start 47.81 47.115) (end 46.4 48.525) (width 0.25) (layer "F.Cu") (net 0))
 (segment (start 47.81 45) (end 47.81 47.115) (width 0.25) (layer "F.Cu") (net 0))
 (segment (start 26.19 47.115) (end 27.6 48.525) (width 0.25) (layer "F.Cu") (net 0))
 (segment (start 45.27 25) (end 44 26.27) (width 0.25) (layer "F.Cu") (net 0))
 (segment (start 40.19 25) (end 40.19 27.115) (width 0.25) (layer "F.Cu") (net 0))
 (segment (start 40.19 27.115) (end 41.6 28.525) (width 0.25) (layer "F.Cu") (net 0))
 (segment (start 47.81 25) (end 47.81 27.115) (width 0.25) (layer "F.Cu") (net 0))
 (segment (start 47.81 27.115) (end 46.4 28.525) (width 0.25) (layer "F.Cu") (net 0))
 (segment (start 42.73 28.455) (end 42.8 28.525) (width 0.25) (layer "F.Cu") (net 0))
 (segment (start 44 26.27) (end 44 28.525) (width 0.25) (layer "F.Cu") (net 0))
 (segment (start 42.73 25) (end 42.73 28.455) (width 0.25) (layer "F.Cu") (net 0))
 (segment (start 26.19 27.115) (end 27.6 28.525) (width 0.25) (layer "F.Cu") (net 1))
 (segment (start 26.19 25) (end 26.19 27.115) (width 0.25) (layer "F.Cu") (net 1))
 (segment (start 33.81 27.115) (end 32.4 28.525) (width 0.25) (layer "F.Cu") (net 5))
 (segment (start 33.81 25) (end 33.81 27.115) (width 0.25) (layer "F.Cu") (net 5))
 (segment (start 30 26.27) (end 30 28.525) (width 0.25) (layer "F.Cu") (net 3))
 (segment (start 31.27 25) (end 30 26.27) (width 0.25) (layer "F.Cu") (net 3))
 (segment (start 28.73 28.455) (end 28.8 28.525) (width 0.25) (layer "F.Cu") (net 2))
 (segment (start 28.73 25) (end 28.73 28.455) (width 0.25) (layer "F.Cu") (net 2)))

